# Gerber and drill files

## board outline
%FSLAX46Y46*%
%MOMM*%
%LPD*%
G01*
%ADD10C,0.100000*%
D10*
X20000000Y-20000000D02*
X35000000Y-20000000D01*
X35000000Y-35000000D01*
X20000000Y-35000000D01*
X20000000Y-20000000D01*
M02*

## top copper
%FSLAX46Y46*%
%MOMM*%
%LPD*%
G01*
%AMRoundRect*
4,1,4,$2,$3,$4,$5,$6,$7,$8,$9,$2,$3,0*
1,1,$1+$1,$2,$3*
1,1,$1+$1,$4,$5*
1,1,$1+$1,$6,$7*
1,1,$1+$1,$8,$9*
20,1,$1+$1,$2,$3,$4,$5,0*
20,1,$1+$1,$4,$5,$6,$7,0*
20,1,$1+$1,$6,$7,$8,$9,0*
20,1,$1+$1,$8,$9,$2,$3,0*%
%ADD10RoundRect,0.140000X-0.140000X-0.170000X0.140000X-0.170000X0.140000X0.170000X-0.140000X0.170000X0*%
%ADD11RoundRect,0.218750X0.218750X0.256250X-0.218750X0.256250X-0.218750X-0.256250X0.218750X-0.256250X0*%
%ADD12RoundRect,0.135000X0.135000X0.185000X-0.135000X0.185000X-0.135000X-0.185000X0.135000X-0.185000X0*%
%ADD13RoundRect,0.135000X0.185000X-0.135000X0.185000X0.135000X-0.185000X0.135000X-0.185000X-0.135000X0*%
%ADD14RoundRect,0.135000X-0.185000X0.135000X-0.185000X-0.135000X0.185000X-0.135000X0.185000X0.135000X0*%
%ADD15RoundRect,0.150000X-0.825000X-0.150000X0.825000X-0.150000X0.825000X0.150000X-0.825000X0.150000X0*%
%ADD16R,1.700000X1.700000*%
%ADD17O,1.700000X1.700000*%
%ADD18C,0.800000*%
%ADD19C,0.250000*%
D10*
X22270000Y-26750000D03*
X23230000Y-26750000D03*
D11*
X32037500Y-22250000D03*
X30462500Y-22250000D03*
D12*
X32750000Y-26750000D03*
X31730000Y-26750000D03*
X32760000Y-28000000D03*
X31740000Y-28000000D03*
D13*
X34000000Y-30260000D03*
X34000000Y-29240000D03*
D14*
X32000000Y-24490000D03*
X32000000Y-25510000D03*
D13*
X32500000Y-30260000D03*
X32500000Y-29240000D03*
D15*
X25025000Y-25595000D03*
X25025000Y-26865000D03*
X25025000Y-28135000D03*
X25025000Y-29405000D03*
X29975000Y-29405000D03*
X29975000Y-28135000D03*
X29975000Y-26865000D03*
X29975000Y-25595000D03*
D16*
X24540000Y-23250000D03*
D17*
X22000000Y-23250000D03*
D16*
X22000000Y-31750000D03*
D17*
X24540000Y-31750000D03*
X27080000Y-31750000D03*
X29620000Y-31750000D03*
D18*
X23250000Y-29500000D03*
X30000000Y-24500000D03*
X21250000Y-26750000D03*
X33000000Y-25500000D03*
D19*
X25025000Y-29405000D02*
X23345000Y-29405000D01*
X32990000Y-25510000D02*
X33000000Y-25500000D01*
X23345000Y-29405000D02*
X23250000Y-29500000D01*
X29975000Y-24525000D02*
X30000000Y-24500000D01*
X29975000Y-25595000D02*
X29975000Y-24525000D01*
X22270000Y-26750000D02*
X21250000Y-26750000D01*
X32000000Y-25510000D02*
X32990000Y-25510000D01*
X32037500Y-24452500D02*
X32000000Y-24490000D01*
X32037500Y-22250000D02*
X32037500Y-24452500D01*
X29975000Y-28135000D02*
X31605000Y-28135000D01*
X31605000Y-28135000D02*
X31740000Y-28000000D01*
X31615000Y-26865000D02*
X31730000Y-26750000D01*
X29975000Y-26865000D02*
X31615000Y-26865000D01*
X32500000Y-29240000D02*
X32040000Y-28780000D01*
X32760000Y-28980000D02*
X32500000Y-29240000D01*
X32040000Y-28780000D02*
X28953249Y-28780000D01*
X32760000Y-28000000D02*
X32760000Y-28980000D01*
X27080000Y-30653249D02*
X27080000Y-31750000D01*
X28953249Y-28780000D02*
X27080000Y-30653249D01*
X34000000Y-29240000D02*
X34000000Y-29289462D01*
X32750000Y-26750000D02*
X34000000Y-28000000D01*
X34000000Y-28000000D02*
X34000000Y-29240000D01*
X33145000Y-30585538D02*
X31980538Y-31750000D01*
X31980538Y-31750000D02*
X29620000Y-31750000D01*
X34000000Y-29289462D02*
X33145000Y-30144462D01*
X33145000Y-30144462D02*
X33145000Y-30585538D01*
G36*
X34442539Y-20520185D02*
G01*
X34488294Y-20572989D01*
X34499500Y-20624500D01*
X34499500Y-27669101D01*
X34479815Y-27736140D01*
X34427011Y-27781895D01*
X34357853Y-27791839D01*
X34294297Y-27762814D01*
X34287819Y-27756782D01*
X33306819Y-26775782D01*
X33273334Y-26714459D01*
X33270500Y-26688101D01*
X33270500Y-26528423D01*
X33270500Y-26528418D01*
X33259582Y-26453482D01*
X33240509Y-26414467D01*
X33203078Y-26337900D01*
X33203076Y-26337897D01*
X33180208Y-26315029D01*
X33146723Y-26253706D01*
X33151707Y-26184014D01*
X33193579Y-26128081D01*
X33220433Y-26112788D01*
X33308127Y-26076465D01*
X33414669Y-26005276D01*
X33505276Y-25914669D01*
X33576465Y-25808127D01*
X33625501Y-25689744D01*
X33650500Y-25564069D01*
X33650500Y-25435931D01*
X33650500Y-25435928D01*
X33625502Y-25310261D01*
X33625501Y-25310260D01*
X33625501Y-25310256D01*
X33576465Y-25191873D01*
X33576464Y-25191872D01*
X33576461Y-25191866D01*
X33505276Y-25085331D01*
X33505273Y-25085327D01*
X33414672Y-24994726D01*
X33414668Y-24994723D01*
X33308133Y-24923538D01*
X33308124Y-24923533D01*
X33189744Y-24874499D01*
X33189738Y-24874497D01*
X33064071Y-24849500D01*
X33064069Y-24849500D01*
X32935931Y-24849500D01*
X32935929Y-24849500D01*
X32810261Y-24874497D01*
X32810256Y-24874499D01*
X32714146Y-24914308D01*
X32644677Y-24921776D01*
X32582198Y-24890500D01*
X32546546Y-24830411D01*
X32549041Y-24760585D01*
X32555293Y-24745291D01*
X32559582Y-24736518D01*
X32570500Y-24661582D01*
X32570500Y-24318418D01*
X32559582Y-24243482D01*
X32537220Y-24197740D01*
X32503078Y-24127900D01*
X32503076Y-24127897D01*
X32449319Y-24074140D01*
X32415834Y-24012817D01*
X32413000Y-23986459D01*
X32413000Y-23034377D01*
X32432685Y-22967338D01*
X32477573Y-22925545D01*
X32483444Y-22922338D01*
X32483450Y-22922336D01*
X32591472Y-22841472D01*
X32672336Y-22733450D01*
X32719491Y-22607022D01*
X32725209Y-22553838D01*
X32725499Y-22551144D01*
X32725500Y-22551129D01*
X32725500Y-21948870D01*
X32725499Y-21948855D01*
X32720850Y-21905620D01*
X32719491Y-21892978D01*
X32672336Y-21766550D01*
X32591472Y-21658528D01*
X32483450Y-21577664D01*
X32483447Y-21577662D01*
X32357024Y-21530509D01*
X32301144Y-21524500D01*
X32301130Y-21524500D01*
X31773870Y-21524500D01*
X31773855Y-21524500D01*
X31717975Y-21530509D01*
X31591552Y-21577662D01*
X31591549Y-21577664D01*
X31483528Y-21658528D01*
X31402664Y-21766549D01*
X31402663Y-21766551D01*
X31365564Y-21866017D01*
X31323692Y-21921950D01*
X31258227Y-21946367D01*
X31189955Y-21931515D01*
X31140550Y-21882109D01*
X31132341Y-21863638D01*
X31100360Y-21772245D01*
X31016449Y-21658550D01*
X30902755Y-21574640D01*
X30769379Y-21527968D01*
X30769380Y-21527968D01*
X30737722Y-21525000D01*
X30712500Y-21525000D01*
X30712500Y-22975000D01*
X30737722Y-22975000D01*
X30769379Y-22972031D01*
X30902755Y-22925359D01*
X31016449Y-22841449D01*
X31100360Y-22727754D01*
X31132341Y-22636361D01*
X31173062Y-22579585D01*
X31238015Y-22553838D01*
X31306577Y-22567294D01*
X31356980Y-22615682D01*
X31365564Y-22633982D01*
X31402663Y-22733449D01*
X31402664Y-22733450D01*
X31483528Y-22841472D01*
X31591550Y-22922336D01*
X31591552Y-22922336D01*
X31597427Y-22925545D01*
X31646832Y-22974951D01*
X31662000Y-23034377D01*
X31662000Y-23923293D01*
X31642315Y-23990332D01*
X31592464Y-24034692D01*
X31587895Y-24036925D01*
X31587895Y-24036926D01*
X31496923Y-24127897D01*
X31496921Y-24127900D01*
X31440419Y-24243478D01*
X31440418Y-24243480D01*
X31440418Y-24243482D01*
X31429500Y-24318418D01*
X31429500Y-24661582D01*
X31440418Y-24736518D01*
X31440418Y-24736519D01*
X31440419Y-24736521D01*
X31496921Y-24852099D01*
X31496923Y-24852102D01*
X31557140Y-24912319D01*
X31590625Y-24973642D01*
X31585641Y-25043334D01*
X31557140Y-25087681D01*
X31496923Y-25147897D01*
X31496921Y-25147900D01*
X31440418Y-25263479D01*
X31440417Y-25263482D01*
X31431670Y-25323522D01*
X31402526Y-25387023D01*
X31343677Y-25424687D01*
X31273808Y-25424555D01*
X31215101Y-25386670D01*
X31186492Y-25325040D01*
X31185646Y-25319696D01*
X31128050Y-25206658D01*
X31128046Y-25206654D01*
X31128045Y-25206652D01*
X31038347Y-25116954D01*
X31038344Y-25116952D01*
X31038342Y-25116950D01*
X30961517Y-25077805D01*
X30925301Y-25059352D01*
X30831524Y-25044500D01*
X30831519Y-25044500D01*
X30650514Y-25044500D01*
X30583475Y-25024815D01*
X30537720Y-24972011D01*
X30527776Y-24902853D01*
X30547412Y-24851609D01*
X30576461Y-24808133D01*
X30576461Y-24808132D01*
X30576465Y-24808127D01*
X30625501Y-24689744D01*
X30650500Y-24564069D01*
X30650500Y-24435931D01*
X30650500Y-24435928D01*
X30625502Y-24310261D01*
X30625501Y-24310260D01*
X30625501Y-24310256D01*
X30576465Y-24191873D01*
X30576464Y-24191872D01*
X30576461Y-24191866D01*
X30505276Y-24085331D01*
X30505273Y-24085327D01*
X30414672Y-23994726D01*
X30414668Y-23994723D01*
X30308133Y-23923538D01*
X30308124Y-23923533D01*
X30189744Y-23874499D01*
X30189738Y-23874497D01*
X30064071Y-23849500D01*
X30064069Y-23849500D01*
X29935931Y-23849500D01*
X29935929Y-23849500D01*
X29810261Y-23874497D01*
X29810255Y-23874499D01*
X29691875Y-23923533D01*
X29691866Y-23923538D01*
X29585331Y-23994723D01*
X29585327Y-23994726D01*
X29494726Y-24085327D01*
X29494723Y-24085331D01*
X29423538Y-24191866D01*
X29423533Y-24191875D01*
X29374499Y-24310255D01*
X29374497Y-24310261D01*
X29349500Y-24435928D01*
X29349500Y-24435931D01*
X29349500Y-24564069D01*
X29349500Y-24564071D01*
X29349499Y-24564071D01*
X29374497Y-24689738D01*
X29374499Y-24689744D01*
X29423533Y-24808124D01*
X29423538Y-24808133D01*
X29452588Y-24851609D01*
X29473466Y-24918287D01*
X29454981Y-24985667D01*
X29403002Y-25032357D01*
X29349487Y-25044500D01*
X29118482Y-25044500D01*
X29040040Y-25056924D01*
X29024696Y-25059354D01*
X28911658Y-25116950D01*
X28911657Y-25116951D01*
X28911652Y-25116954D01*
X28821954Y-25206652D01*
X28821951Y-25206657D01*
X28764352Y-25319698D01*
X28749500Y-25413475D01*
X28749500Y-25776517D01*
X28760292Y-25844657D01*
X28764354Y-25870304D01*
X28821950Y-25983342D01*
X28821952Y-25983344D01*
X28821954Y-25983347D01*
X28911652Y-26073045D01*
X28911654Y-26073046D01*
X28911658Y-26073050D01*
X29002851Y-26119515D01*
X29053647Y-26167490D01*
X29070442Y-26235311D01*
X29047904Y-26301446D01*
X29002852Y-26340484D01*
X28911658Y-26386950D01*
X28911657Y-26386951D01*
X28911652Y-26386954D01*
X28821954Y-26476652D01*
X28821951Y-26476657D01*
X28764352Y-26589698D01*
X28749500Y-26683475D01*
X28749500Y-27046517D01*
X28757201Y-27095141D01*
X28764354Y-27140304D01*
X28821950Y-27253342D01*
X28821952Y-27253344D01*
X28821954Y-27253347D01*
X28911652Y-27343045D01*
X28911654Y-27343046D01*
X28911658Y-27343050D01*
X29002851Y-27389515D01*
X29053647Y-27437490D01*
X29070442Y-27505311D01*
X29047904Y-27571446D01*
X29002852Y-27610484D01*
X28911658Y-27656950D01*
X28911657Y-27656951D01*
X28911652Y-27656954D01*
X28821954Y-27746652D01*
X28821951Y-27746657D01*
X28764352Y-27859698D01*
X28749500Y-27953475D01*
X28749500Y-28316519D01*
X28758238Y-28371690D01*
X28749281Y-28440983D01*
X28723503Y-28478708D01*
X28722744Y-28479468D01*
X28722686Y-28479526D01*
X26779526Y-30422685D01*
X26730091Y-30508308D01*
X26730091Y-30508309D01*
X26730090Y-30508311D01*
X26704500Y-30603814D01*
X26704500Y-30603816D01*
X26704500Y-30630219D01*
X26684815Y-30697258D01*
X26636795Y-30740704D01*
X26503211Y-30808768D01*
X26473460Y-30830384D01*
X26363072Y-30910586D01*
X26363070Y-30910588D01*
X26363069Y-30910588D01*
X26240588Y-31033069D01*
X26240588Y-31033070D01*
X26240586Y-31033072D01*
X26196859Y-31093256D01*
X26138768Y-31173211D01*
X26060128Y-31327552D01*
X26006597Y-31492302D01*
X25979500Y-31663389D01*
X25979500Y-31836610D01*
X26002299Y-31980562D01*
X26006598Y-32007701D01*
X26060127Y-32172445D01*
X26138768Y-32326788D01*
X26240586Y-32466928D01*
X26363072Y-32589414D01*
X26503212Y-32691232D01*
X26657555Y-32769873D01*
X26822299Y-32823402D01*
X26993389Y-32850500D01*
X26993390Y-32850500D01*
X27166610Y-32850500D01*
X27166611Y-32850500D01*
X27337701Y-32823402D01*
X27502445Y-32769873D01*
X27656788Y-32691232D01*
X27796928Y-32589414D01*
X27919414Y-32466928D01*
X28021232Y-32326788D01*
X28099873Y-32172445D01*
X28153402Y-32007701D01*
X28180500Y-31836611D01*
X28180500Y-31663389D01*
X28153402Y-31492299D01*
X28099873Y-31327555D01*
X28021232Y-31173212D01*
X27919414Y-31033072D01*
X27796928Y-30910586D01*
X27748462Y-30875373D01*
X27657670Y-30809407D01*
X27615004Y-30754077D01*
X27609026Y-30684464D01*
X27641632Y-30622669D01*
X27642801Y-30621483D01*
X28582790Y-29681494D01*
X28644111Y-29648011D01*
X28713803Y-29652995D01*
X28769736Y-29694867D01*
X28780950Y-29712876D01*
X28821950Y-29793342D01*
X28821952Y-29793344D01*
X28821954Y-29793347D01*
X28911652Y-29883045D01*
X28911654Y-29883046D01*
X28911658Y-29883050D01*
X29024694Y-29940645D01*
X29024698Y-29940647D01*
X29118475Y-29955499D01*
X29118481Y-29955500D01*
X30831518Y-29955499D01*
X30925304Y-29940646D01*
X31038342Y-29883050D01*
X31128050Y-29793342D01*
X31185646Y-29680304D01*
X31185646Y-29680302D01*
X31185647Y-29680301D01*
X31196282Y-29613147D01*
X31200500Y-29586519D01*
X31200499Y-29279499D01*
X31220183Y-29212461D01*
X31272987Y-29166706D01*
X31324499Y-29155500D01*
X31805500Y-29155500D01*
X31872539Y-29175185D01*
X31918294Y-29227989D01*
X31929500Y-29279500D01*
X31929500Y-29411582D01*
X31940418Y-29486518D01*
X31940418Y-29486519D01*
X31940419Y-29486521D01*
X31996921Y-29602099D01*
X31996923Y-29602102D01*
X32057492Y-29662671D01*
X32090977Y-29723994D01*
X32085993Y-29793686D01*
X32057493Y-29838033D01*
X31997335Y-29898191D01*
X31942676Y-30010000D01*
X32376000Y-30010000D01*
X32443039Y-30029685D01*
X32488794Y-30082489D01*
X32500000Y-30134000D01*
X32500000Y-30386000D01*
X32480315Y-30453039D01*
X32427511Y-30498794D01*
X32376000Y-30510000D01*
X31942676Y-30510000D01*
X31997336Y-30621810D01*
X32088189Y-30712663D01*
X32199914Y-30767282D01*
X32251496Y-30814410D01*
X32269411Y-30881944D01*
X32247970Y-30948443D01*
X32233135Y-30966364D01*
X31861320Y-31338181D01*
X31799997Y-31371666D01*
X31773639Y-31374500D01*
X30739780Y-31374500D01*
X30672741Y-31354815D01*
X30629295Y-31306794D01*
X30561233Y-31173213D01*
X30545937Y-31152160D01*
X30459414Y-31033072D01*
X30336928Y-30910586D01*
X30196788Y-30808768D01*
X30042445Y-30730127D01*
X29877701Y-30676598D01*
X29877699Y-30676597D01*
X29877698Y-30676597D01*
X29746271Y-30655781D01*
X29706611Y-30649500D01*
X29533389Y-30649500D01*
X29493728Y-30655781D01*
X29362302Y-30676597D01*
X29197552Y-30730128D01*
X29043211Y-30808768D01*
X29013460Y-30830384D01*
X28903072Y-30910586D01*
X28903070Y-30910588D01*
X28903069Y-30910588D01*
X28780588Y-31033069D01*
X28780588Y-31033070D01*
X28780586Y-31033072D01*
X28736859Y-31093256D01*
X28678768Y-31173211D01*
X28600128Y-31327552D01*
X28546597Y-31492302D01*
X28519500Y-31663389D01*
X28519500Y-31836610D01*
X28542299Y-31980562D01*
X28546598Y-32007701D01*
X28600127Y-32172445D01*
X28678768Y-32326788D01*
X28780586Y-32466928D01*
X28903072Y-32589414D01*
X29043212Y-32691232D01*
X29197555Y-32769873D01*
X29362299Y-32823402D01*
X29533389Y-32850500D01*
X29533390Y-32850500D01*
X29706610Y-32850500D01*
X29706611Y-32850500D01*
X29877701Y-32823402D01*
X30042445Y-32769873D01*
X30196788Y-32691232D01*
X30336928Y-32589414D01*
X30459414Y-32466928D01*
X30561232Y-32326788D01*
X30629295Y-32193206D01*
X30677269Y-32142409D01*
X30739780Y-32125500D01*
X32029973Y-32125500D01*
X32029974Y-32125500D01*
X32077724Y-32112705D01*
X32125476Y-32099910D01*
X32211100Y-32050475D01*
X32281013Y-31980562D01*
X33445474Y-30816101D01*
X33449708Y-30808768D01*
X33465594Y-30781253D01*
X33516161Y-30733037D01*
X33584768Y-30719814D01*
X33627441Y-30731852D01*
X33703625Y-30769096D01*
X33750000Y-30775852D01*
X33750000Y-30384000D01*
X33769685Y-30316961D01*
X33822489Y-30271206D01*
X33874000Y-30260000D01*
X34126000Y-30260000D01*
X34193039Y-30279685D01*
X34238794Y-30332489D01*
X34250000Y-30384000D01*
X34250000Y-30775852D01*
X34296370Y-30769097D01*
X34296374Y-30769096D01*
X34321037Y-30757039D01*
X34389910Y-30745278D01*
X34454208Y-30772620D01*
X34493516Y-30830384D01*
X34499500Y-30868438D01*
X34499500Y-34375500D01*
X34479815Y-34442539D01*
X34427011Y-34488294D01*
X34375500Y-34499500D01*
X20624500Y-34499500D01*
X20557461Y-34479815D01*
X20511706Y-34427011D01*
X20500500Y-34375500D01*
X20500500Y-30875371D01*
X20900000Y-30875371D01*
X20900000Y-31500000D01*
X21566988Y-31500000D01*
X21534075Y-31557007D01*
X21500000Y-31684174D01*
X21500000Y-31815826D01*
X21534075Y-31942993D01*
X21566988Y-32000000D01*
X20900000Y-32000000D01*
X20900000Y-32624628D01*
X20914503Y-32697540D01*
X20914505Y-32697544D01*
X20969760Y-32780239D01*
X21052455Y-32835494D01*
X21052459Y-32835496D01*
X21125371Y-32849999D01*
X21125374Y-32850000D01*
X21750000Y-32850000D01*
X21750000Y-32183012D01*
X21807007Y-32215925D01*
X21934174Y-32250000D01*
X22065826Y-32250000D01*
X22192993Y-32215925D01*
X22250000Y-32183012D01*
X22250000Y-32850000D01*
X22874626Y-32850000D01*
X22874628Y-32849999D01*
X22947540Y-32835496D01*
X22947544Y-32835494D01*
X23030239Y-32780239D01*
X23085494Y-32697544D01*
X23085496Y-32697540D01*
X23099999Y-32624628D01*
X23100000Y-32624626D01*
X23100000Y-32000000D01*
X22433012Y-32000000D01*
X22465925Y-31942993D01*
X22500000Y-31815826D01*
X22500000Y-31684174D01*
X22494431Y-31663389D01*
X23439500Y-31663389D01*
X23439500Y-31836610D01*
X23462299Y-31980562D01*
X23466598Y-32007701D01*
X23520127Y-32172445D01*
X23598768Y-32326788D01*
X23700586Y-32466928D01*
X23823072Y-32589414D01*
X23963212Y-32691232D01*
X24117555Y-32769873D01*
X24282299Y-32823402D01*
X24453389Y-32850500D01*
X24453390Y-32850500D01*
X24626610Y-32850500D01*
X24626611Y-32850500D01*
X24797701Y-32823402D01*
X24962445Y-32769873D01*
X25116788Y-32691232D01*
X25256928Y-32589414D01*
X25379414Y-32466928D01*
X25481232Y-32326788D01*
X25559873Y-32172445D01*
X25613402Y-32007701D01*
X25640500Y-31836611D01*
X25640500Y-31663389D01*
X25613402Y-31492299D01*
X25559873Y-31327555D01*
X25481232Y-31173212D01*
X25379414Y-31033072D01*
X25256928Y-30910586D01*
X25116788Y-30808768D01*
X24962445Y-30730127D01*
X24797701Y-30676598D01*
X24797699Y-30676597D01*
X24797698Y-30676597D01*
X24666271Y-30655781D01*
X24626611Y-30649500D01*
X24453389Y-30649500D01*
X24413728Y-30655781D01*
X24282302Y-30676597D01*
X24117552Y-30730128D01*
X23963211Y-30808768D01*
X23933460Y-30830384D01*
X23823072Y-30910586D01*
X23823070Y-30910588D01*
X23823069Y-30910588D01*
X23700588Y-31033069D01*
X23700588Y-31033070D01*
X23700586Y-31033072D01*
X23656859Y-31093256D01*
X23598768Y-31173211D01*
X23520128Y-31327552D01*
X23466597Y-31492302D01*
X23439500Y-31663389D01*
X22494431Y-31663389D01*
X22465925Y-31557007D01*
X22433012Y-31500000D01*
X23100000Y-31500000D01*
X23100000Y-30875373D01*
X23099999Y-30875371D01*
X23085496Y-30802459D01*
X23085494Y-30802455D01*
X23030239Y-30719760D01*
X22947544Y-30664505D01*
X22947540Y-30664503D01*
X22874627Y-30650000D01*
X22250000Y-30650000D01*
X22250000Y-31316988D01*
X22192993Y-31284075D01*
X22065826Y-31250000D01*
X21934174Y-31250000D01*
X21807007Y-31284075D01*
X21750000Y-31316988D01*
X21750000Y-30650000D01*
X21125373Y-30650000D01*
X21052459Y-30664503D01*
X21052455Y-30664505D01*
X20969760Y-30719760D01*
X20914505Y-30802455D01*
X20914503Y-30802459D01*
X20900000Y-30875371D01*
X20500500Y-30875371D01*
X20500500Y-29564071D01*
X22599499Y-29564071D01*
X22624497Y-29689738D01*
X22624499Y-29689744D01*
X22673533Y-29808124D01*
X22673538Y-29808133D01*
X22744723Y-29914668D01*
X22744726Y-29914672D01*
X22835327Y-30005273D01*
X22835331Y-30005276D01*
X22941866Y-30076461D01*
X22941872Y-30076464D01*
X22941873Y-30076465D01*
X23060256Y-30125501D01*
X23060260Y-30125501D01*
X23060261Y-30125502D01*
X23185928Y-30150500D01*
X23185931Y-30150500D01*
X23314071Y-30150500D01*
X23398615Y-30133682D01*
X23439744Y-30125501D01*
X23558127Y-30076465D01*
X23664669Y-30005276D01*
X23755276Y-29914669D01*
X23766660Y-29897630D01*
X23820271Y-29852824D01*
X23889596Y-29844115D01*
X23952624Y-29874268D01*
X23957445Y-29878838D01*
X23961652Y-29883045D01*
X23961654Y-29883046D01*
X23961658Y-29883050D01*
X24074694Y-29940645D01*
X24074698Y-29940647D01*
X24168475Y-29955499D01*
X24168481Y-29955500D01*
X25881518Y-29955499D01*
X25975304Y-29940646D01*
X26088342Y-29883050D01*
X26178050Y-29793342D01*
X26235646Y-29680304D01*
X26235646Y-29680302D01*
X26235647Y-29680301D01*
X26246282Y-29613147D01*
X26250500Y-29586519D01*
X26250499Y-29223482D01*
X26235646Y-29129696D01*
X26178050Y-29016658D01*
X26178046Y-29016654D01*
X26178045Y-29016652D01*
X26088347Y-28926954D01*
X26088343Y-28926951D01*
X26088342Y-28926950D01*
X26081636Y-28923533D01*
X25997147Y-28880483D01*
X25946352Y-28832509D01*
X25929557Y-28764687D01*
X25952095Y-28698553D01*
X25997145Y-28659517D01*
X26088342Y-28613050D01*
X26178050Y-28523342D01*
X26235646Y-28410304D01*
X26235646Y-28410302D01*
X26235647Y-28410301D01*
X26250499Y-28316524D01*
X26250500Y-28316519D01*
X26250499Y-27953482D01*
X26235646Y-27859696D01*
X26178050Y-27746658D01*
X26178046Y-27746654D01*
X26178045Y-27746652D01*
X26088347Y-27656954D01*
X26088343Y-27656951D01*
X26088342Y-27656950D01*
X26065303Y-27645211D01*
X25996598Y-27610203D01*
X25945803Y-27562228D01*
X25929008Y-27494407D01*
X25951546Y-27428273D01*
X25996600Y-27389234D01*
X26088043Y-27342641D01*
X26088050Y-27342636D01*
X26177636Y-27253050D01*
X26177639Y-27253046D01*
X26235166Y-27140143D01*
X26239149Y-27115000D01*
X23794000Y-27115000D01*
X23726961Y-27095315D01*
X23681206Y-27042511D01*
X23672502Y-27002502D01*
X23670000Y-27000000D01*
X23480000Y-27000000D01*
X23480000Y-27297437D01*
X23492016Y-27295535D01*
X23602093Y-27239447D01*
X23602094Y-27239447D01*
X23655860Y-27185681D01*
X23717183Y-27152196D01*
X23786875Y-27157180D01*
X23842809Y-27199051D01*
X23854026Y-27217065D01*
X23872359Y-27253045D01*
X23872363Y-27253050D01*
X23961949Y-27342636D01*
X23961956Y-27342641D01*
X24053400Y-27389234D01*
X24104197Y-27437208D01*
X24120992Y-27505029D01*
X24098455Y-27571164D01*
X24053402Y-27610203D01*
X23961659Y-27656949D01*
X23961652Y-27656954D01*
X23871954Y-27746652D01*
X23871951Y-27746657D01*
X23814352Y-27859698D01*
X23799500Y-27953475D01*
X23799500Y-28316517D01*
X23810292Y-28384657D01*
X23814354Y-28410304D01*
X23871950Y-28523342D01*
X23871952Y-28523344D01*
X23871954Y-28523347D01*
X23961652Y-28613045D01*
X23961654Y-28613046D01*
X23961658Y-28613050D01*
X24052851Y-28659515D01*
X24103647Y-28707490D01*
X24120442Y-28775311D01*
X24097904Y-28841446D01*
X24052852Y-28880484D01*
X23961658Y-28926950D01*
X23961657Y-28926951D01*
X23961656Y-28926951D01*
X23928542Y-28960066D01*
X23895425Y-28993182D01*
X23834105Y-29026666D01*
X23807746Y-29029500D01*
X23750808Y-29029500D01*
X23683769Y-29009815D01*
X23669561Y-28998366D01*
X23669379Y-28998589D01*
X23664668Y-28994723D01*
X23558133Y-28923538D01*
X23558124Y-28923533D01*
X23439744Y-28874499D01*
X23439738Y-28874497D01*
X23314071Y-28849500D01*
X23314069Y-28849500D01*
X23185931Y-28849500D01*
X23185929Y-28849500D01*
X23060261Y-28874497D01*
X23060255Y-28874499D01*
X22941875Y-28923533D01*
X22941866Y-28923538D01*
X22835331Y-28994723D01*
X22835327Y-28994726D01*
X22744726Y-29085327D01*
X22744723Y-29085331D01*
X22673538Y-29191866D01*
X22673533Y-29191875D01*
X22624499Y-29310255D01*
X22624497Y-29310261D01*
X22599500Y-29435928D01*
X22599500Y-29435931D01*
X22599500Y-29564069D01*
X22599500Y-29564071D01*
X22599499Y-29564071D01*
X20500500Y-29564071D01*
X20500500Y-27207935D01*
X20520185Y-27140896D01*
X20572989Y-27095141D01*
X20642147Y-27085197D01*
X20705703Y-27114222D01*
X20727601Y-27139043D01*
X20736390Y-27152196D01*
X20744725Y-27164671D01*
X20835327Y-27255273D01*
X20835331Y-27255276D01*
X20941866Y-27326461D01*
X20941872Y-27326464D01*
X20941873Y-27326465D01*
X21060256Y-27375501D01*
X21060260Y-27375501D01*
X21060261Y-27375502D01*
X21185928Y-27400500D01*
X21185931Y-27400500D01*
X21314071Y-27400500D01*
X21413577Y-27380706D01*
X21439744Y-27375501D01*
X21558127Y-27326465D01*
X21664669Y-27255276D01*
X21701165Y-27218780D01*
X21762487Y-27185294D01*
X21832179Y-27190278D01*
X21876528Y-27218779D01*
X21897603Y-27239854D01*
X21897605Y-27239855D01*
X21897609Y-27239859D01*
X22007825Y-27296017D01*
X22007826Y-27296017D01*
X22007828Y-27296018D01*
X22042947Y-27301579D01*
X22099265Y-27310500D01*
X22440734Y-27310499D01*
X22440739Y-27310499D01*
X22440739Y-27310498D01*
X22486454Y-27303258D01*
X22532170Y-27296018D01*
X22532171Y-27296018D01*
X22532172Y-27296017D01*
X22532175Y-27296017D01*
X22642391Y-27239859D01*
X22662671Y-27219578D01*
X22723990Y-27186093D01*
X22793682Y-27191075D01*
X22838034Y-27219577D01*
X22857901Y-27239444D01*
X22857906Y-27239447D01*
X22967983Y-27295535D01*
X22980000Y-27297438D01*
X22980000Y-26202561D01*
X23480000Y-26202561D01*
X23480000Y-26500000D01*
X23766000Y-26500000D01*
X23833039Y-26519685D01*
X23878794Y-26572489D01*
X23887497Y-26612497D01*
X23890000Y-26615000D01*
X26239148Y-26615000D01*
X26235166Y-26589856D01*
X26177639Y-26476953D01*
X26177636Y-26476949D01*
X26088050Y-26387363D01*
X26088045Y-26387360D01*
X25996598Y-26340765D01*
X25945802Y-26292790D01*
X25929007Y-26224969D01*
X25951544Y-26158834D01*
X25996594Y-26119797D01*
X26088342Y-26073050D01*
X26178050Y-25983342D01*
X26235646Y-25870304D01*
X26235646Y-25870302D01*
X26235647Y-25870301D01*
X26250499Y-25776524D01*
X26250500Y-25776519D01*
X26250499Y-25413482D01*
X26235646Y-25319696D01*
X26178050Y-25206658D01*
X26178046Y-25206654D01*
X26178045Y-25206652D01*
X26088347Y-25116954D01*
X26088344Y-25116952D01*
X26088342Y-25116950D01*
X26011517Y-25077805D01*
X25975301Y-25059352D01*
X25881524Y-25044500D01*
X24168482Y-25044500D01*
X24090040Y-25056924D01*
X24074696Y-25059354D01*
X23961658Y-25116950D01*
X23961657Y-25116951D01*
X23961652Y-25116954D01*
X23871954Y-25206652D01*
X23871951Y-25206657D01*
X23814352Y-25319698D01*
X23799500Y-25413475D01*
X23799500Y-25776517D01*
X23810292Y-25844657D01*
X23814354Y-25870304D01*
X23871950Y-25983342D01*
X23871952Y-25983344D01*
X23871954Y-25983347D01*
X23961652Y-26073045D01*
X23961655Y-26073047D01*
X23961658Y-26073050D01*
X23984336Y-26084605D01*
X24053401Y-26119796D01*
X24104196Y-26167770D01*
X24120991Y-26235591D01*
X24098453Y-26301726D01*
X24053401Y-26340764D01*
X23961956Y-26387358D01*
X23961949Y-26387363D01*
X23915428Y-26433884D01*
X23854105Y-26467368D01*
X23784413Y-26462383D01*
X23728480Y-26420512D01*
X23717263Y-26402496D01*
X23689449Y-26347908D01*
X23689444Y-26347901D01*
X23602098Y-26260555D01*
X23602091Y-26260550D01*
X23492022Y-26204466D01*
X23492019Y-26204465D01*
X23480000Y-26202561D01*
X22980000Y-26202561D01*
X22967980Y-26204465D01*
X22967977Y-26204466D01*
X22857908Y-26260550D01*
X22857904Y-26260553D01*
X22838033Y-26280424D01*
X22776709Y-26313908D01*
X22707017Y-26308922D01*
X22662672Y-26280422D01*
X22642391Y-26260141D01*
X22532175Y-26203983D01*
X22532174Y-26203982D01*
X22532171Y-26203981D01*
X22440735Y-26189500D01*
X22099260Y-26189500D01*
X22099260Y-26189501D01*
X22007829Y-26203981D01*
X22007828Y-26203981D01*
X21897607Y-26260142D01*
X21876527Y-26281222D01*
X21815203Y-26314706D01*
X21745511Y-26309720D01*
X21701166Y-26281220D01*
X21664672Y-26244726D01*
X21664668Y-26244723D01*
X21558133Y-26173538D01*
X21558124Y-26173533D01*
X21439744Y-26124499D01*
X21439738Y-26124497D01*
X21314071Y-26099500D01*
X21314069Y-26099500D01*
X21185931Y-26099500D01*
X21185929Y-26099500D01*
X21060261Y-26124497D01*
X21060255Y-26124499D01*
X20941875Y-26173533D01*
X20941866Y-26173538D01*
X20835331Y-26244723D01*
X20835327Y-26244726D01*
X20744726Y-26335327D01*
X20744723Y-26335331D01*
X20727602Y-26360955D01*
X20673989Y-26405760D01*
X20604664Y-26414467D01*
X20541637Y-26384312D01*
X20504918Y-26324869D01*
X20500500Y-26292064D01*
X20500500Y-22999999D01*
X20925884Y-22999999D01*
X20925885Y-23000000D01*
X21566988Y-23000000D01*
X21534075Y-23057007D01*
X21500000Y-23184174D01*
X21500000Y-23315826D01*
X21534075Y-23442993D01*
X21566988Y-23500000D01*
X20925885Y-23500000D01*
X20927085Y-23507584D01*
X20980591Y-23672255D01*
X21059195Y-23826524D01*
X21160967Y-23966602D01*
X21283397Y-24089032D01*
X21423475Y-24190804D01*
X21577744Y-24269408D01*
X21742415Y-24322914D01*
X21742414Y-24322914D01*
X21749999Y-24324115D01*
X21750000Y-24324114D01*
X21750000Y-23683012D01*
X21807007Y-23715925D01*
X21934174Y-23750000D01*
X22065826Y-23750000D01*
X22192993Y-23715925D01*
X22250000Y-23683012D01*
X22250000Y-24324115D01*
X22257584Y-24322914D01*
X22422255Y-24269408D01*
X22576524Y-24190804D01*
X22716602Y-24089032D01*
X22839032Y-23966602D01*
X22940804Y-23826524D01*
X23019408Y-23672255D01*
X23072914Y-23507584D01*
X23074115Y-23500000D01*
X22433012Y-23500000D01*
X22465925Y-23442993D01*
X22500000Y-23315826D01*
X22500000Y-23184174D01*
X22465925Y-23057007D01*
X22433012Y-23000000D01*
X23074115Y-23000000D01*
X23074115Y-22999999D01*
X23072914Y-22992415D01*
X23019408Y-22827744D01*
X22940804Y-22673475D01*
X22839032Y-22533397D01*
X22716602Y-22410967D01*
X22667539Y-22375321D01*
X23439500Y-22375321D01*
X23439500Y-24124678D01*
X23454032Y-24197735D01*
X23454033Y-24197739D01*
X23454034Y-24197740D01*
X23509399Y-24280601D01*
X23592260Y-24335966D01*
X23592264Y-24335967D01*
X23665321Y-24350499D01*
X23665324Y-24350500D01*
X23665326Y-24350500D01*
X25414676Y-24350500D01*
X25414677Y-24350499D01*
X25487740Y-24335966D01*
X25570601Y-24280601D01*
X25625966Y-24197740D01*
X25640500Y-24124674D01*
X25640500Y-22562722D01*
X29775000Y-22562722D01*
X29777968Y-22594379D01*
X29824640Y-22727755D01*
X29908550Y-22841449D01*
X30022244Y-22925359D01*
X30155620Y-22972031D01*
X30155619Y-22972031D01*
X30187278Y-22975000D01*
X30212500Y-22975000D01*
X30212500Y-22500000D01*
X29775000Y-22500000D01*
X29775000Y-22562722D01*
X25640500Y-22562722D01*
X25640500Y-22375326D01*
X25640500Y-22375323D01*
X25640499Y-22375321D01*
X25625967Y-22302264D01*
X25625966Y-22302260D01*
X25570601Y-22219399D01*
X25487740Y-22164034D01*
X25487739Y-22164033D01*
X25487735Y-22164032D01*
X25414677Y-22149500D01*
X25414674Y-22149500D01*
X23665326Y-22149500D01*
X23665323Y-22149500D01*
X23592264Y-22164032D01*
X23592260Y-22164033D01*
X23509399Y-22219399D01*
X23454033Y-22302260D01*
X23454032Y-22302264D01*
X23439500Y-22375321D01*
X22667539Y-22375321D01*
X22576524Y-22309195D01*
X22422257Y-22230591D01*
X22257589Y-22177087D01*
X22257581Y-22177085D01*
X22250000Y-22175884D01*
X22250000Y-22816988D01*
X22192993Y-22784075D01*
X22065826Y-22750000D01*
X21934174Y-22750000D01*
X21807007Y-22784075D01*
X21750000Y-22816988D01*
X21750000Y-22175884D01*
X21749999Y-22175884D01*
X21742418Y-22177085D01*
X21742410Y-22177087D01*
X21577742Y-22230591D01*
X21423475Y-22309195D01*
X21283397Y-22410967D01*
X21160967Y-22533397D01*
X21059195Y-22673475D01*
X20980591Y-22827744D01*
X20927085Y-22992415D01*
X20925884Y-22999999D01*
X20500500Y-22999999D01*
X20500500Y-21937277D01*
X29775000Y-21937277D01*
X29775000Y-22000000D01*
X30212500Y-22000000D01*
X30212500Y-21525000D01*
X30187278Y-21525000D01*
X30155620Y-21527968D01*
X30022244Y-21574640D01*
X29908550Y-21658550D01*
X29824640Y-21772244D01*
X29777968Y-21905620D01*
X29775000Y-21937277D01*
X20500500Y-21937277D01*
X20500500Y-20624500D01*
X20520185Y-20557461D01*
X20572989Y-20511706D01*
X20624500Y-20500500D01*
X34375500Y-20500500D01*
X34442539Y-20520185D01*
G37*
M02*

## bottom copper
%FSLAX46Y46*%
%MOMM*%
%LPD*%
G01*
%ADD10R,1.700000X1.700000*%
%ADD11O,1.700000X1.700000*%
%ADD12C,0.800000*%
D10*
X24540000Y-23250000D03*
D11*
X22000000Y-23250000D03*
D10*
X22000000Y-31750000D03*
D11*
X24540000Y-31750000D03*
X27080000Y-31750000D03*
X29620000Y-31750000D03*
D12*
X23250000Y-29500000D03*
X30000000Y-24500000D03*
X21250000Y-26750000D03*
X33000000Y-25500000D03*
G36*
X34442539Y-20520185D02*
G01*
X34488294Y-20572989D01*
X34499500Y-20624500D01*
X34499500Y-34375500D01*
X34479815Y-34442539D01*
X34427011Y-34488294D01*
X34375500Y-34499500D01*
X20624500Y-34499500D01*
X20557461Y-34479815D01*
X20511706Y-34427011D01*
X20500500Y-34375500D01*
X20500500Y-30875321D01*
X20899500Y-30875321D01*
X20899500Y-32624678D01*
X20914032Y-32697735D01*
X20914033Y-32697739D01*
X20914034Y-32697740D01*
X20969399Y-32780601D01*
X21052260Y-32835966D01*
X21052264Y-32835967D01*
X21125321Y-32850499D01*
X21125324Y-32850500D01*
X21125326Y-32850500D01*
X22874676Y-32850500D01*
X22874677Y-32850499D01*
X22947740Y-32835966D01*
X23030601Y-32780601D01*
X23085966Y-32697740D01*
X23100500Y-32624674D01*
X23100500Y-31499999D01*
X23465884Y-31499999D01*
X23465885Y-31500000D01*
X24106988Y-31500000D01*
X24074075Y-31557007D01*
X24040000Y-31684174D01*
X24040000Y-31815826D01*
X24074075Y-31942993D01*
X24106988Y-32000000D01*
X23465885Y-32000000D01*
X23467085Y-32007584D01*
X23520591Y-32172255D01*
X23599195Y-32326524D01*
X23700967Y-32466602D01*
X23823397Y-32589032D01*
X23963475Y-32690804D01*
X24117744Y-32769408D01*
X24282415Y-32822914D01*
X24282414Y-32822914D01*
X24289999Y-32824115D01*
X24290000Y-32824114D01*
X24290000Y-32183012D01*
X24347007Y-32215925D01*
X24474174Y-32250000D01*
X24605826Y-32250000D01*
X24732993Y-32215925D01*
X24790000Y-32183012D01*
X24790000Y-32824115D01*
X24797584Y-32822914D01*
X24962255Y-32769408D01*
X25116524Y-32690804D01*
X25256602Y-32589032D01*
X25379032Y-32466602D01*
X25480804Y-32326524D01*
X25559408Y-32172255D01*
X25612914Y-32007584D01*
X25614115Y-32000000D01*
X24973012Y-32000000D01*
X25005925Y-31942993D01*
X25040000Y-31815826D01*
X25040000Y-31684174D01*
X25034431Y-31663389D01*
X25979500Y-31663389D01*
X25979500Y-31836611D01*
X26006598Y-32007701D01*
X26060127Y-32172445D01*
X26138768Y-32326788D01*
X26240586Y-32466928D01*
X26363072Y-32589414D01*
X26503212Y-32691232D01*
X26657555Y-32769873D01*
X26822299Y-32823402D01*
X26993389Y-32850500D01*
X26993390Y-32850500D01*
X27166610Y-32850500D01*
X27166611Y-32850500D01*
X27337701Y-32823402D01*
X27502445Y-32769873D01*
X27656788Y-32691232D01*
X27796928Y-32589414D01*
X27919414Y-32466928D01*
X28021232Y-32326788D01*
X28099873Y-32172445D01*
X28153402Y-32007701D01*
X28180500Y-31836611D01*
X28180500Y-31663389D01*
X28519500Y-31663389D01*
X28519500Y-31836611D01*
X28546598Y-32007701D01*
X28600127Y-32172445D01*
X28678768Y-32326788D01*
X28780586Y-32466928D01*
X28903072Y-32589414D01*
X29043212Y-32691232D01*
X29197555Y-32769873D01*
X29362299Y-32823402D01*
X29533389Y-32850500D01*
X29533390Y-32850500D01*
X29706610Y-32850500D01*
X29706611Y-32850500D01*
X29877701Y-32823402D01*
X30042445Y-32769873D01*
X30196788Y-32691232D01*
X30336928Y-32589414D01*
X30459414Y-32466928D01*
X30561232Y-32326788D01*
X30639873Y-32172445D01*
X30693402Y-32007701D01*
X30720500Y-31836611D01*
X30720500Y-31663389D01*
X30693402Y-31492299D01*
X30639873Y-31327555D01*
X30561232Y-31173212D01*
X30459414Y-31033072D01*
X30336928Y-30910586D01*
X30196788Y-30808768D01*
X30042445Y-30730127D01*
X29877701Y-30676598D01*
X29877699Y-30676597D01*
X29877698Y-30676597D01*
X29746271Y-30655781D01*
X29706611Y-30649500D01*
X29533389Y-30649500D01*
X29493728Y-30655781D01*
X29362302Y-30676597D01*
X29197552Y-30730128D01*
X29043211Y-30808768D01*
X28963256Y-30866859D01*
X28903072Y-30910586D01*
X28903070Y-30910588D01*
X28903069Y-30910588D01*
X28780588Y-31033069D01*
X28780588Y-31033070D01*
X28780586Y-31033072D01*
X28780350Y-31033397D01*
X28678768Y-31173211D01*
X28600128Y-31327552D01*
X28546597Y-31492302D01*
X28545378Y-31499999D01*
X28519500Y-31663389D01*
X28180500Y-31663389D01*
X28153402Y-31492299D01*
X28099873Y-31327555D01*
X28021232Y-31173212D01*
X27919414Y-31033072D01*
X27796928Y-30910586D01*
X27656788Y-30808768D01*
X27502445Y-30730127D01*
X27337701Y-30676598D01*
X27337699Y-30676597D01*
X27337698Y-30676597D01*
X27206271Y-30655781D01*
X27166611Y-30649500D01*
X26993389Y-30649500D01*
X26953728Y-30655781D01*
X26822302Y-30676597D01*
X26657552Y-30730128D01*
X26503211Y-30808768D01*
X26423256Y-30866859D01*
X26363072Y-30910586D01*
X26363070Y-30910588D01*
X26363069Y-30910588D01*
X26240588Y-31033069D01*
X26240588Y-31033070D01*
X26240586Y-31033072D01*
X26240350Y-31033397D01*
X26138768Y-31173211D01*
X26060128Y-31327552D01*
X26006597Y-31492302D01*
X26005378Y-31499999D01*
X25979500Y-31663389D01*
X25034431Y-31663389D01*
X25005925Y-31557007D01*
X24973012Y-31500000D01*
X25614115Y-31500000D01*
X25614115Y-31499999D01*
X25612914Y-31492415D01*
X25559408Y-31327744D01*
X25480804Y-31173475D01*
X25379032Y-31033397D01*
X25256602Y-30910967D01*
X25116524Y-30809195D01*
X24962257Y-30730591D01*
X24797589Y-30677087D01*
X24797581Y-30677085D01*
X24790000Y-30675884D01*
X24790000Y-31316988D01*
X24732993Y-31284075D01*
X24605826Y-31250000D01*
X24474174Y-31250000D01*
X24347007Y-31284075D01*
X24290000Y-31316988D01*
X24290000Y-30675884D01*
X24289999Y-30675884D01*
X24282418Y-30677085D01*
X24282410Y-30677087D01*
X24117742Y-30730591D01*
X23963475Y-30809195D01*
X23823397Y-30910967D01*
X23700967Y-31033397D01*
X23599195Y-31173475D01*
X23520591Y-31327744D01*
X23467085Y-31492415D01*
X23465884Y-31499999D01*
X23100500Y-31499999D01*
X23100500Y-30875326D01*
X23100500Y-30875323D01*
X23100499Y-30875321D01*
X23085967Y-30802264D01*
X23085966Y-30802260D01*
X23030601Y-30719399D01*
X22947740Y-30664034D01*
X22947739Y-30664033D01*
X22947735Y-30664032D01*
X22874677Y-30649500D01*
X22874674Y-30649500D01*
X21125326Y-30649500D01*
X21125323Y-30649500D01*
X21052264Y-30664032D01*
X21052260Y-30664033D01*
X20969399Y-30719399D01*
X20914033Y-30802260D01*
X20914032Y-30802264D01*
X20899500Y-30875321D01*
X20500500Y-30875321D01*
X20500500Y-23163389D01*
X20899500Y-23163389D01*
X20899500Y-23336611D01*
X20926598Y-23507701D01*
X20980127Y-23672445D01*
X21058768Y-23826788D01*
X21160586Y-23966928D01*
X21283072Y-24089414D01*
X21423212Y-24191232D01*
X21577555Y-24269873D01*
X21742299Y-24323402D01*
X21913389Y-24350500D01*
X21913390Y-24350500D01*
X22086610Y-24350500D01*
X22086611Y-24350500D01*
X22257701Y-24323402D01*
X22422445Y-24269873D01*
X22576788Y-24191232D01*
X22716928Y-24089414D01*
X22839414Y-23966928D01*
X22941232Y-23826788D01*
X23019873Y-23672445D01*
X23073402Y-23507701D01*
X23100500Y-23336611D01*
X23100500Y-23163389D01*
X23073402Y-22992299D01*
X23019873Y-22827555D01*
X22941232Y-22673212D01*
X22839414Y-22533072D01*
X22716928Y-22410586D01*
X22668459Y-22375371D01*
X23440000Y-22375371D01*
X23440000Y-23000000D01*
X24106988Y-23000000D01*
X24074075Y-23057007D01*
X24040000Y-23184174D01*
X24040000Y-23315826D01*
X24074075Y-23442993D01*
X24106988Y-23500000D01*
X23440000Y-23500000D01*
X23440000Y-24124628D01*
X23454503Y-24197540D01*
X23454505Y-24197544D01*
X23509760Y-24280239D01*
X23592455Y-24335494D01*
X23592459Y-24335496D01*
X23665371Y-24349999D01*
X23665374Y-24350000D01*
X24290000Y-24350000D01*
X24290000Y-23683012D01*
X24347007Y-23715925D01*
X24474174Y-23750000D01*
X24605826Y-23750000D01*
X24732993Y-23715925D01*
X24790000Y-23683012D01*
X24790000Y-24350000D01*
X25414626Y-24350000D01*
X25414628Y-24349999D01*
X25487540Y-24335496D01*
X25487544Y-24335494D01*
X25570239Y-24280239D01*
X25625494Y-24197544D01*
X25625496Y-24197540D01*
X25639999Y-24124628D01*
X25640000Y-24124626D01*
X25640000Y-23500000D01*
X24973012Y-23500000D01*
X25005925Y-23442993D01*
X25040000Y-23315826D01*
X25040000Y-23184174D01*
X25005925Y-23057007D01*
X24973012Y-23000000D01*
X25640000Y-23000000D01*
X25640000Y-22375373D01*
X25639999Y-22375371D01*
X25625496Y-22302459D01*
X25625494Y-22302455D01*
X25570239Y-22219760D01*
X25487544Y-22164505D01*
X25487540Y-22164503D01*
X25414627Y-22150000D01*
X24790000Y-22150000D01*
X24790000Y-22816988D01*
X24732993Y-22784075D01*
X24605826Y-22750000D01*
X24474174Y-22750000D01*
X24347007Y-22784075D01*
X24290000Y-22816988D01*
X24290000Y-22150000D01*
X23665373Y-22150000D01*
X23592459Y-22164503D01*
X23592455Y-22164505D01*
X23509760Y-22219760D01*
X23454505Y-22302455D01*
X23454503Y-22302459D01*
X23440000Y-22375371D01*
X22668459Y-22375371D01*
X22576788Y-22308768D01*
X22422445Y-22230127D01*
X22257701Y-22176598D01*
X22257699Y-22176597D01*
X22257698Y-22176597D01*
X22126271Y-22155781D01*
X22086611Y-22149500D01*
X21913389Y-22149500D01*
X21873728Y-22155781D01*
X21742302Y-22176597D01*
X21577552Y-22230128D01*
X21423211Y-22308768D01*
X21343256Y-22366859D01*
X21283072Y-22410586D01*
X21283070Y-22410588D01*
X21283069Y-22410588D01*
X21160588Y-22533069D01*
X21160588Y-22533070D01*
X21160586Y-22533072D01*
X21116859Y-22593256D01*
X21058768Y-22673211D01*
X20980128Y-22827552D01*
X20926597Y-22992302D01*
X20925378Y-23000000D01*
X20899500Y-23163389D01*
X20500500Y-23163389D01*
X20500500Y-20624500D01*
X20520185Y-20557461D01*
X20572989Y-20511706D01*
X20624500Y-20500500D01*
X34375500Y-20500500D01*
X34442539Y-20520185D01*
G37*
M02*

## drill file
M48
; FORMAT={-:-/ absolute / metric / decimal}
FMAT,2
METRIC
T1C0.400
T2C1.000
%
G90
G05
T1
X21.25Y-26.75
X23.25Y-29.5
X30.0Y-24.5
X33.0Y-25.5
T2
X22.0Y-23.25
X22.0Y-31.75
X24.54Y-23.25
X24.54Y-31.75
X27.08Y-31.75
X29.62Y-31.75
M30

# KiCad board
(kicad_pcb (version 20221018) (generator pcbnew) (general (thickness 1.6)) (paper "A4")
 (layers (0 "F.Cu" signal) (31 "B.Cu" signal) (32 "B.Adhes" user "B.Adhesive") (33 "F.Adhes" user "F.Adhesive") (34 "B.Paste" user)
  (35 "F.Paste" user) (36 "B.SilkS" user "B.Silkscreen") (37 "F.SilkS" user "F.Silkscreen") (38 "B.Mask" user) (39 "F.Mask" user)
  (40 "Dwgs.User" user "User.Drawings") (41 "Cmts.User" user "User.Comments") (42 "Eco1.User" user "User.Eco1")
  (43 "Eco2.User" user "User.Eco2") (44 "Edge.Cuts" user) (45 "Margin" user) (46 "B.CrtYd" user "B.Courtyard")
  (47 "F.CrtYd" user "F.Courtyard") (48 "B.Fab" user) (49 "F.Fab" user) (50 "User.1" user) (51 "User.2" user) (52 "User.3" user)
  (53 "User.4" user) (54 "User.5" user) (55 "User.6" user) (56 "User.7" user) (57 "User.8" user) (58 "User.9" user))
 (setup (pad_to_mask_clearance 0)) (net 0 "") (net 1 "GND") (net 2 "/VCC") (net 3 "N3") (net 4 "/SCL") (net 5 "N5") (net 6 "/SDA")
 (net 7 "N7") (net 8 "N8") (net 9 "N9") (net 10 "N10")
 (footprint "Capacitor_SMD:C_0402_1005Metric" (layer "F.Cu") (at 22.75 26.75)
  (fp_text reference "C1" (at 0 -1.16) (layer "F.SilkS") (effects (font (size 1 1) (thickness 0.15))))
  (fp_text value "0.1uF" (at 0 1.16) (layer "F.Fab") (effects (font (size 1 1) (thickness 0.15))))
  (pad "1" smd roundrect (at -0.48 0) (size 0.56 0.62) (layers "F.Cu" "F.Paste" "F.Mask") (roundrect_rratio 0.25) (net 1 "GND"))
  (pad "2" smd roundrect (at 0.48 0) (size 0.56 0.62) (layers "F.Cu" "F.Paste" "F.Mask") (roundrect_rratio 0.25) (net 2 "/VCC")))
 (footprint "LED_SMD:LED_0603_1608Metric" (layer "F.Cu") (at 31.25 22.25 180)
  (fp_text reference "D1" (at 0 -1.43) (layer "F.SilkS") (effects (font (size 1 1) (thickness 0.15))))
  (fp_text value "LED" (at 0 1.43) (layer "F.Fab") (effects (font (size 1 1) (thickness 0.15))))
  (pad "1" smd roundrect (at -0.7875 0 180) (size 0.875 0.95) (layers "F.Cu" "F.Paste" "F.Mask") (roundrect_rratio 0.25) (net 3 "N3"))
  (pad "2" smd roundrect (at 0.7875 0 180) (size 0.875 0.95) (layers "F.Cu" "F.Paste" "F.Mask") (roundrect_rratio 0.25) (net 2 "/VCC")))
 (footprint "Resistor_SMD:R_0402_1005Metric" (layer "F.Cu") (at 32.24 26.75 180)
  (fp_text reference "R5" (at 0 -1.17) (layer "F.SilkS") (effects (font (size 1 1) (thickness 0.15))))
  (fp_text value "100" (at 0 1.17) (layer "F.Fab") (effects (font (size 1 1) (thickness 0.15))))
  (pad "1" smd roundrect (at -0.51 0 180) (size 0.54 0.64) (layers "F.Cu" "F.Paste" "F.Mask") (roundrect_rratio 0.25) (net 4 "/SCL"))
  (pad "2" smd roundrect (at 0.51 0 180) (size 0.54 0.64) (layers "F.Cu" "F.Paste" "F.Mask") (roundrect_rratio 0.25) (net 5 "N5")))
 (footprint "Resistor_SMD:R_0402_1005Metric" (layer "F.Cu") (at 32.25 28 180)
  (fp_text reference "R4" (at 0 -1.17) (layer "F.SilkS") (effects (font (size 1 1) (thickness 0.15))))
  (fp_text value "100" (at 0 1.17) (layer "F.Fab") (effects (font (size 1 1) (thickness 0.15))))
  (pad "1" smd roundrect (at -0.51 0 180) (size 0.54 0.64) (layers "F.Cu" "F.Paste" "F.Mask") (roundrect_rratio 0.25) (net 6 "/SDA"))
  (pad "2" smd roundrect (at 0.51 0 180) (size 0.54 0.64) (layers "F.Cu" "F.Paste" "F.Mask") (roundrect_rratio 0.25) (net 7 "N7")))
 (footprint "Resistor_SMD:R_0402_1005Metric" (layer "F.Cu") (at 34 29.75 90)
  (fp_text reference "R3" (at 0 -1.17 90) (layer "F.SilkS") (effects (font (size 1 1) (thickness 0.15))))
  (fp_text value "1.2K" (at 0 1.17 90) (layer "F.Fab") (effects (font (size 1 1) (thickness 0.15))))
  (pad "1" smd roundrect (at -0.51 0 90) (size 0.54 0.64) (layers "F.Cu" "F.Paste" "F.Mask") (roundrect_rratio 0.25) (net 2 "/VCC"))
  (pad "2" smd roundrect (at 0.51 0 90) (size 0.54 0.64) (layers "F.Cu" "F.Paste" "F.Mask") (roundrect_rratio 0.25) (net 4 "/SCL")))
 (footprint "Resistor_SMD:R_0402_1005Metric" (layer "F.Cu") (at 32 25 -90)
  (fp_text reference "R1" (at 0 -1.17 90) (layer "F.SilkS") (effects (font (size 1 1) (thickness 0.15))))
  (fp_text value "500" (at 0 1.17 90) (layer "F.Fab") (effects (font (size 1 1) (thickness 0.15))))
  (pad "1" smd roundrect (at -0.51 0 270) (size 0.54 0.64) (layers "F.Cu" "F.Paste" "F.Mask") (roundrect_rratio 0.25) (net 3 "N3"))
  (pad "2" smd roundrect (at 0.51 0 270) (size 0.54 0.64) (layers "F.Cu" "F.Paste" "F.Mask") (roundrect_rratio 0.25) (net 1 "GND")))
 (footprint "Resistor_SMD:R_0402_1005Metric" (layer "F.Cu") (at 32.5 29.75 90)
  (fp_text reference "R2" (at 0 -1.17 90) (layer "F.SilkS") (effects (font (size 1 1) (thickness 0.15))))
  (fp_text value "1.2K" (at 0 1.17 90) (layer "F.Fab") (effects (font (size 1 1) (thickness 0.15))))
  (pad "1" smd roundrect (at -0.51 0 90) (size 0.54 0.64) (layers "F.Cu" "F.Paste" "F.Mask") (roundrect_rratio 0.25) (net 2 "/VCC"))
  (pad "2" smd roundrect (at 0.51 0 90) (size 0.54 0.64) (layers "F.Cu" "F.Paste" "F.Mask") (roundrect_rratio 0.25) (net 6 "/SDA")))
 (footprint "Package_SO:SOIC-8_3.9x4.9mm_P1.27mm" (layer "F.Cu") (at 27.5 27.5)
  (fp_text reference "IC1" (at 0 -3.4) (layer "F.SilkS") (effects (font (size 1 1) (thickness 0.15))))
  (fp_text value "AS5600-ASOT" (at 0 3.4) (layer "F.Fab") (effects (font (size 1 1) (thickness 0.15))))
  (pad "1" smd roundrect (at -2.475 -1.905) (size 1.95 0.6) (layers "F.Cu" "F.Paste" "F.Mask") (roundrect_rratio 0.25) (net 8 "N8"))
  (pad "2" smd roundrect (at -2.475 -0.635) (size 1.95 0.6) (layers "F.Cu" "F.Paste" "F.Mask") (roundrect_rratio 0.25) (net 2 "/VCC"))
  (pad "3" smd roundrect (at -2.475 0.635) (size 1.95 0.6) (layers "F.Cu" "F.Paste" "F.Mask") (roundrect_rratio 0.25) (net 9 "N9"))
  (pad "4" smd roundrect (at -2.475 1.905) (size 1.95 0.6) (layers "F.Cu" "F.Paste" "F.Mask") (roundrect_rratio 0.25) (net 1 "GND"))
  (pad "5" smd roundrect (at 2.475 1.905) (size 1.95 0.6) (layers "F.Cu" "F.Paste" "F.Mask") (roundrect_rratio 0.25) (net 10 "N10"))
  (pad "6" smd roundrect (at 2.475 0.635) (size 1.95 0.6) (layers "F.Cu" "F.Paste" "F.Mask") (roundrect_rratio 0.25) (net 7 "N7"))
  (pad "7" smd roundrect (at 2.475 -0.635) (size 1.95 0.6) (layers "F.Cu" "F.Paste" "F.Mask") (roundrect_rratio 0.25) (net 5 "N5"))
  (pad "8" smd roundrect (at 2.475 -1.905) (size 1.95 0.6) (layers "F.Cu" "F.Paste" "F.Mask") (roundrect_rratio 0.25) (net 1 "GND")))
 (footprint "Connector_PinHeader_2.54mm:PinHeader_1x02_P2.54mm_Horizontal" (layer "B.Cu") (at 24.54 23.25 90)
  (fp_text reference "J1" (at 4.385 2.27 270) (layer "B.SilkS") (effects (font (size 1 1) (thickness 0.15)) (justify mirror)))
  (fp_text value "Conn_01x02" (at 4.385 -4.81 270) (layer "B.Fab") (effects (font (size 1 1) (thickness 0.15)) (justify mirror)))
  (pad "1" thru_hole rect (at 0 0 90) (size 1.7 1.7) (drill 1) (layers "*.Cu" "*.Mask") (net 1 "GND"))
  (pad "2" thru_hole oval (at 0 -2.54 90) (size 1.7 1.7) (drill 1) (layers "*.Cu" "*.Mask") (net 2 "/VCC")))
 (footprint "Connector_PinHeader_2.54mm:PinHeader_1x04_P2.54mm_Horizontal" (layer "B.Cu") (at 22 31.75 -90)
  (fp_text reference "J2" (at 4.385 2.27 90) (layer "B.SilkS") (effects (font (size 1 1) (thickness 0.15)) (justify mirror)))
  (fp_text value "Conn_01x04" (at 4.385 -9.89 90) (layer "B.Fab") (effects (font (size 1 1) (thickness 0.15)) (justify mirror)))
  (pad "1" thru_hole rect (at 0 0 270) (size 1.7 1.7) (drill 1) (layers "*.Cu" "*.Mask") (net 2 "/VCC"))
  (pad "2" thru_hole oval (at 0 -2.54 270) (size 1.7 1.7) (drill 1) (layers "*.Cu" "*.Mask") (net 1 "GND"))
  (pad "3" thru_hole oval (at 0 -5.08 270) (size 1.7 1.7) (drill 1) (layers "*.Cu" "*.Mask") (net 6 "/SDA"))
  (pad "4" thru_hole oval (at 0 -7.62 270) (size 1.7 1.7) (drill 1) (layers "*.Cu" "*.Mask") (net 4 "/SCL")))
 (gr_rect (start 20 20) (end 35 35) (stroke (width 0.1) (type default)) (fill none) (layer "Edge.Cuts"))
 (segment (start 25.025 29.405) (end 23.345 29.405) (width 0.25) (layer "F.Cu") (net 1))
 (segment (start 32.99 25.51) (end 33 25.5) (width 0.25) (layer "F.Cu") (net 1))
 (segment (start 23.345 29.405) (end 23.25 29.5) (width 0.25) (layer "F.Cu") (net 1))
 (segment (start 29.975 24.525) (end 30 24.5) (width 0.25) (layer "F.Cu") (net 1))
 (segment (start 29.975 25.595) (end 29.975 24.525) (width 0.25) (layer "F.Cu") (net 1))
 (segment (start 22.27 26.75) (end 21.25 26.75) (width 0.25) (layer "F.Cu") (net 1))
 (segment (start 32 25.51) (end 32.99 25.51) (width 0.25) (layer "F.Cu") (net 1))
 (via (at 23.25 29.5) (size 0.8) (drill 0.4) (layers "F.Cu" "B.Cu") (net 1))
 (via (at 30 24.5) (size 0.8) (drill 0.4) (layers "F.Cu" "B.Cu") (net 1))
 (via (at 21.25 26.75) (size 0.8) (drill 0.4) (layers "F.Cu" "B.Cu") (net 1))
 (via (at 33 25.5) (size 0.8) (drill 0.4) (layers "F.Cu" "B.Cu") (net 1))
 (segment (start 32.0375 24.4525) (end 32 24.49) (width 0.25) (layer "F.Cu") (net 3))
 (segment (start 32.0375 22.25) (end 32.0375 24.4525) (width 0.25) (layer "F.Cu") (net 3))
 (segment (start 29.975 28.135) (end 31.605 28.135) (width 0.25) (layer "F.Cu") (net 7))
 (segment (start 31.605 28.135) (end 31.74 28) (width 0.25) (layer "F.Cu") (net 7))
 (segment (start 31.615 26.865) (end 31.73 26.75) (width 0.25) (layer "F.Cu") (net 5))
 (segment (start 29.975 26.865) (end 31.615 26.865) (width 0.25) (layer "F.Cu") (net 5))
 (segment (start 32.5 29.24) (end 32.04 28.78) (width 0.25) (layer "F.Cu") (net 6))
 (segment (start 32.76 28.98) (end 32.5 29.24) (width 0.25) (layer "F.Cu") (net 6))
 (segment (start 32.04 28.78) (end 28.953249 28.78) (width 0.25) (layer "F.Cu") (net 6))
 (segment (start 32.76 28) (end 32.76 28.98) (width 0.25) (layer "F.Cu") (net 6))
 (segment (start 27.08 30.653249) (end 27.08 31.75) (width 0.25) (layer "F.Cu") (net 6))
 (segment (start 28.953249 28.78) (end 27.08 30.653249) (width 0.25) (layer "F.Cu") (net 6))
 (segment (start 34 29.24) (end 34 29.289462) (width 0.25) (layer "F.Cu") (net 4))
 (segment (start 32.75 26.75) (end 34 28) (width 0.25) (layer "F.Cu") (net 4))
 (segment (start 34 28) (end 34 29.24) (width 0.25) (layer "F.Cu") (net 4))
 (segment (start 33.145 30.585538) (end 31.980538 31.75) (width 0.25) (layer "F.Cu") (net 4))
 (segment (start 31.980538 31.75) (end 29.62 31.75) (width 0.25) (layer "F.Cu") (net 4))
 (segment (start 34 29.289462) (end 33.145 30.144462) (width 0.25) (layer "F.Cu") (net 4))
 (segment (start 33.145 30.144462) (end 33.145 30.585538) (width 0.25) (layer "F.Cu") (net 4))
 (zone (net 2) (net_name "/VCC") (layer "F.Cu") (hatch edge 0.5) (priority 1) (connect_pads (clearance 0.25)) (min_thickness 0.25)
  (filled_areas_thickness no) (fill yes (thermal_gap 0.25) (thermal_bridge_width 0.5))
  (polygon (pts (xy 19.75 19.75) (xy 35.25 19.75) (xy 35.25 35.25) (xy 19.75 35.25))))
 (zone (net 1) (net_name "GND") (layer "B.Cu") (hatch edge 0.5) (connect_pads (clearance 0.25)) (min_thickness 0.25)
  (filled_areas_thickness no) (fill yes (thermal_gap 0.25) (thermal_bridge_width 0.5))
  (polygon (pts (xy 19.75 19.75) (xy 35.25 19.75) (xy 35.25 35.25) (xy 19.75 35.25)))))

